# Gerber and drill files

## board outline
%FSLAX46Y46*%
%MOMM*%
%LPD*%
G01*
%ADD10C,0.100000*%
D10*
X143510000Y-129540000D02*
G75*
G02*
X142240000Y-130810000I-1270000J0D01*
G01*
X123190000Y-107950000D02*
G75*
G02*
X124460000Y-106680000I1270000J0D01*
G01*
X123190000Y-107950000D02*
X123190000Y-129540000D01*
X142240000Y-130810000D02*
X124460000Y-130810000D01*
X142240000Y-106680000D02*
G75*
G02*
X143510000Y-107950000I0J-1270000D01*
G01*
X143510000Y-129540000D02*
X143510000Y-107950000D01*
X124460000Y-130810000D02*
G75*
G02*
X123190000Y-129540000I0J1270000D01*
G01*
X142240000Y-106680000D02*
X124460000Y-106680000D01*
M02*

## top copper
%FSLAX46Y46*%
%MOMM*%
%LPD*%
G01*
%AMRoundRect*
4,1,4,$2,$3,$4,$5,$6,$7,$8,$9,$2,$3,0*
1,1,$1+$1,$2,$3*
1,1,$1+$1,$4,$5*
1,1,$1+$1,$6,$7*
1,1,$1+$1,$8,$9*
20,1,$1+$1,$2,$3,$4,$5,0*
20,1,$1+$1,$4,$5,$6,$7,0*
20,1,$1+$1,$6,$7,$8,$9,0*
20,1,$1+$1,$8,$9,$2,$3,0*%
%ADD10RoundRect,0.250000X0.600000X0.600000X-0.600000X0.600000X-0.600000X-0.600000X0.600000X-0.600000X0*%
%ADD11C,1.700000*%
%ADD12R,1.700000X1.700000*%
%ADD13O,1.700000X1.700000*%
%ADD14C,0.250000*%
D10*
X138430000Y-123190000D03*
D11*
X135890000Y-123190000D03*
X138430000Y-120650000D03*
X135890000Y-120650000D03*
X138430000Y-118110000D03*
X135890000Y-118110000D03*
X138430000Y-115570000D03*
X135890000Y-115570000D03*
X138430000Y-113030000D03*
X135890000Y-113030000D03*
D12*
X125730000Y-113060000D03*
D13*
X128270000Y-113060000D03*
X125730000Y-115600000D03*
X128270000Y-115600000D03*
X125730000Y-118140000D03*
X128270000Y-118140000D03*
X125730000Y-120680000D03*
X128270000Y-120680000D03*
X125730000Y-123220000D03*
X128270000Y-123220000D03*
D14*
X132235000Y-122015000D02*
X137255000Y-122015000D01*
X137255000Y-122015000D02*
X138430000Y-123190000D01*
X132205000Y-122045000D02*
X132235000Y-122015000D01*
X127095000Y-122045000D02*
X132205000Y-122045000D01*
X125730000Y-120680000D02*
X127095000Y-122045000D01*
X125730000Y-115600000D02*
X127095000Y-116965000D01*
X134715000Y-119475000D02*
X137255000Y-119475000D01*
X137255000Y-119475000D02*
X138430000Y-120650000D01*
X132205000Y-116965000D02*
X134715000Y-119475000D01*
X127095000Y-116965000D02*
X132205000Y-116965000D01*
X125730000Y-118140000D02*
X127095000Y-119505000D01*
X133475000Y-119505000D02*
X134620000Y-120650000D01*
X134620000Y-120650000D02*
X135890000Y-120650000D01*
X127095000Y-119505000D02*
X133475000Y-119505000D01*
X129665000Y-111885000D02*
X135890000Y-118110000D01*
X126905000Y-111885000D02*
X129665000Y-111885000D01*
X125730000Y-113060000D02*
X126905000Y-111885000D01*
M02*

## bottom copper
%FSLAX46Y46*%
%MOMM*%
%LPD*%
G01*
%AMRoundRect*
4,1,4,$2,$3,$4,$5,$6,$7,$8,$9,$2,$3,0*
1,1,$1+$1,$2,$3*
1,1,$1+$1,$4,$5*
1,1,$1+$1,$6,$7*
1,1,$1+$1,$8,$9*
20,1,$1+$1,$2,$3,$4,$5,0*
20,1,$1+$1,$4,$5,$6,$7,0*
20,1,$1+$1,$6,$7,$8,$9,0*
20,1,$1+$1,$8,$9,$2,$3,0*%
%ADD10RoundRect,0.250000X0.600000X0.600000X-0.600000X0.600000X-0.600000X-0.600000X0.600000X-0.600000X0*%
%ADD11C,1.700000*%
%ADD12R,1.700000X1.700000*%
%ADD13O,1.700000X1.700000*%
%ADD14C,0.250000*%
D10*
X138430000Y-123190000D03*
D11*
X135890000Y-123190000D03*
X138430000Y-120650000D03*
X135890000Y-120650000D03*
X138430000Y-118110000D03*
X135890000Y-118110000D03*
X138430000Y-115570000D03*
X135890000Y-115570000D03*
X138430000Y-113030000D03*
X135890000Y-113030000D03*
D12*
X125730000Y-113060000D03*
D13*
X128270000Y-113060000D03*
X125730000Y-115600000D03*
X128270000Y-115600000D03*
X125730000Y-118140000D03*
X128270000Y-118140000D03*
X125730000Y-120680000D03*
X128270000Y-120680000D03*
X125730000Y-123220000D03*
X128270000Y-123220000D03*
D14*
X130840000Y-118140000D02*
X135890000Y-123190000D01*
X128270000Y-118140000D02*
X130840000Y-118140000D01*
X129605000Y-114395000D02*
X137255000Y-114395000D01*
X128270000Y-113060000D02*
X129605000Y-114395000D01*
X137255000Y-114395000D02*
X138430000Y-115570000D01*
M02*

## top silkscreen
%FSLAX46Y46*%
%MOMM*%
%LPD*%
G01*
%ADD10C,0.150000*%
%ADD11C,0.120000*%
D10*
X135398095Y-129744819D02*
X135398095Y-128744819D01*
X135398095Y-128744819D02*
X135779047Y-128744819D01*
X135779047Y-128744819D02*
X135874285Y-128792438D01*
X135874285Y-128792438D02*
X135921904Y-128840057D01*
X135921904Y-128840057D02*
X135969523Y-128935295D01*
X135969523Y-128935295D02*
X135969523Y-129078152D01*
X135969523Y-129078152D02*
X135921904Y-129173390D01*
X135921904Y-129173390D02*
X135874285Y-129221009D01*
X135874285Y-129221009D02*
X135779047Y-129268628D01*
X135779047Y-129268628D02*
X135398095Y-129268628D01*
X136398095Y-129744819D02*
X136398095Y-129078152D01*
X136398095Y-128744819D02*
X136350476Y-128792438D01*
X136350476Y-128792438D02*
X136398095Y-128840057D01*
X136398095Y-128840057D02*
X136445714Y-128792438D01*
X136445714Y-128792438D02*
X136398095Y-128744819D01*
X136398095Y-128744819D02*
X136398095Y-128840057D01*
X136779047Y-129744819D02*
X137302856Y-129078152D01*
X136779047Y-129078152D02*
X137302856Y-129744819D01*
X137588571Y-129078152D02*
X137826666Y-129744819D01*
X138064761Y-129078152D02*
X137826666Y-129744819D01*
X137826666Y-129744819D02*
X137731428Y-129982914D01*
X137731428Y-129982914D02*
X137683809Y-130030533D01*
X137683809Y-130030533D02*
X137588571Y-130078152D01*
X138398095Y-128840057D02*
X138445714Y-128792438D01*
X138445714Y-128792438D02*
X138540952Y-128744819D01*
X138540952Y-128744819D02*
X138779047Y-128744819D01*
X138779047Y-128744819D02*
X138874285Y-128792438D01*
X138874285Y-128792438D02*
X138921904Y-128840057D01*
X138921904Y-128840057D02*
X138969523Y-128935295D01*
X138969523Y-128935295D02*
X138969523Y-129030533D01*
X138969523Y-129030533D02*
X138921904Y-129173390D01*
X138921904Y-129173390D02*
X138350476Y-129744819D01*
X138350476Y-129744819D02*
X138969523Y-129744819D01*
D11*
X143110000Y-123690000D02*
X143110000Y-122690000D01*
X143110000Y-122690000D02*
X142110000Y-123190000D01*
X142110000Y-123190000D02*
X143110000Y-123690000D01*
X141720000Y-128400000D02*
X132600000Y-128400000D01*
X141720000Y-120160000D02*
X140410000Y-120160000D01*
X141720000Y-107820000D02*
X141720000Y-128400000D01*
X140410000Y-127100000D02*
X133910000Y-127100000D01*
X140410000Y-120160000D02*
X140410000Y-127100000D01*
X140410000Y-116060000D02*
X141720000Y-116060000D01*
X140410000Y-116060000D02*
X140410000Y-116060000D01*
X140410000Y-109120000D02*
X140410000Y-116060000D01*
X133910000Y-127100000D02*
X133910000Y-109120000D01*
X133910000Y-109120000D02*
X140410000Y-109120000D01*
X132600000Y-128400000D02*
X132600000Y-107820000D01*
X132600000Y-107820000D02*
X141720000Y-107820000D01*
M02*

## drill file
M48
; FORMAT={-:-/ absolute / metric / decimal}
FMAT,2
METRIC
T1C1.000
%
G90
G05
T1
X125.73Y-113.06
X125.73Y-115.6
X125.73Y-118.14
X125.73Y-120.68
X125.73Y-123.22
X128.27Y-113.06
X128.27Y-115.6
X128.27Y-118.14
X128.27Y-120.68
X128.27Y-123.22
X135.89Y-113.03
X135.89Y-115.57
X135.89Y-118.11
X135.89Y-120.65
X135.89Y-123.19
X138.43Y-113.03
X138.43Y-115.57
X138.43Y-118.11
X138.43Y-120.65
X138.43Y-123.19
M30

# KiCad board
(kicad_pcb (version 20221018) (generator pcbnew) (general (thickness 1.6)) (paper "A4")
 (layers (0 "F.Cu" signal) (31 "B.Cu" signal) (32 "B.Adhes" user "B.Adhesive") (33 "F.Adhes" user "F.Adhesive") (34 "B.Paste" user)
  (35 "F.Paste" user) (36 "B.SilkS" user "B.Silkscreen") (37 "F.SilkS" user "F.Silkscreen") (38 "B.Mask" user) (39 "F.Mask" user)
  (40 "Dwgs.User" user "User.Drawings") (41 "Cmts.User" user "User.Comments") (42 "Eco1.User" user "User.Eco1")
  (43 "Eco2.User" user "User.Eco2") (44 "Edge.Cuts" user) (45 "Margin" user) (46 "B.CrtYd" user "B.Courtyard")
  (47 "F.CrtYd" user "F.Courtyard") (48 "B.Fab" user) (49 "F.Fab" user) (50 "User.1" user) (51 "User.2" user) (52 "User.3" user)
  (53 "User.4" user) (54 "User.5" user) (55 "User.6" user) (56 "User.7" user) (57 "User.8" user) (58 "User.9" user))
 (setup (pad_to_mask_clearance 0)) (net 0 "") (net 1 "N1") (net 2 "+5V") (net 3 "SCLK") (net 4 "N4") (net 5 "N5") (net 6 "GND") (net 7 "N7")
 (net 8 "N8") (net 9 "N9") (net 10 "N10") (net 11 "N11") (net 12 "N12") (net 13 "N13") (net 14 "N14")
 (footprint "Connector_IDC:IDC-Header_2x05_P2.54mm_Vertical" (layer "F.Cu") (at 138.43 123.19 180)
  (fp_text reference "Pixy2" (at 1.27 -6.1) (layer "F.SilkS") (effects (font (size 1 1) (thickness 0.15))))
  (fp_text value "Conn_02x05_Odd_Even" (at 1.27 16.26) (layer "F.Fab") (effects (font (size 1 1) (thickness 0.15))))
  (fp_line (start -4.68 -0.5) (end -4.68 0.5) (stroke (width 0.12) (type solid)) (layer "F.SilkS"))
  (fp_line (start -4.68 0.5) (end -3.68 0) (stroke (width 0.12) (type solid)) (layer "F.SilkS"))
  (fp_line (start -3.68 0) (end -4.68 -0.5) (stroke (width 0.12) (type solid)) (layer "F.SilkS"))
  (fp_line (start -3.29 -5.21) (end 5.83 -5.21) (stroke (width 0.12) (type solid)) (layer "F.SilkS"))
  (fp_line (start -3.29 3.03) (end -1.98 3.03) (stroke (width 0.12) (type solid)) (layer "F.SilkS"))
  (fp_line (start -3.29 15.37) (end -3.29 -5.21) (stroke (width 0.12) (type solid)) (layer "F.SilkS"))
  (fp_line (start -1.98 -3.91) (end 4.52 -3.91) (stroke (width 0.12) (type solid)) (layer "F.SilkS"))
  (fp_line (start -1.98 3.03) (end -1.98 -3.91) (stroke (width 0.12) (type solid)) (layer "F.SilkS"))
  (fp_line (start -1.98 7.13) (end -3.29 7.13) (stroke (width 0.12) (type solid)) (layer "F.SilkS"))
  (fp_line (start -1.98 7.13) (end -1.98 7.13) (stroke (width 0.12) (type solid)) (layer "F.SilkS"))
  (fp_line (start -1.98 14.07) (end -1.98 7.13) (stroke (width 0.12) (type solid)) (layer "F.SilkS"))
  (fp_line (start 4.52 -3.91) (end 4.52 14.07) (stroke (width 0.12) (type solid)) (layer "F.SilkS"))
  (fp_line (start 4.52 14.07) (end -1.98 14.07) (stroke (width 0.12) (type solid)) (layer "F.SilkS"))
  (fp_line (start 5.83 -5.21) (end 5.83 15.37) (stroke (width 0.12) (type solid)) (layer "F.SilkS"))
  (fp_line (start 5.83 15.37) (end -3.29 15.37) (stroke (width 0.12) (type solid)) (layer "F.SilkS"))
  (pad "1" thru_hole roundrect (at 0 0 180) (size 1.7 1.7) (drill 1) (layers "*.Cu" "*.Mask") (roundrect_rratio 0.147059) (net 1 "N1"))
  (pad "2" thru_hole circle (at 2.54 0 180) (size 1.7 1.7) (drill 1) (layers "*.Cu" "*.Mask") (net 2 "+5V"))
  (pad "3" thru_hole circle (at 0 2.54 180) (size 1.7 1.7) (drill 1) (layers "*.Cu" "*.Mask") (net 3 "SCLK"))
  (pad "4" thru_hole circle (at 2.54 2.54 180) (size 1.7 1.7) (drill 1) (layers "*.Cu" "*.Mask") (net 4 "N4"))
  (pad "5" thru_hole circle (at 0 5.08 180) (size 1.7 1.7) (drill 1) (layers "*.Cu" "*.Mask") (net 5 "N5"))
  (pad "6" thru_hole circle (at 2.54 5.08 180) (size 1.7 1.7) (drill 1) (layers "*.Cu" "*.Mask") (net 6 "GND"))
  (pad "7" thru_hole circle (at 0 7.62 180) (size 1.7 1.7) (drill 1) (layers "*.Cu" "*.Mask") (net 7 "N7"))
  (pad "8" thru_hole circle (at 2.54 7.62 180) (size 1.7 1.7) (drill 1) (layers "*.Cu" "*.Mask") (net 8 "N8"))
  (pad "9" thru_hole circle (at 0 10.16 180) (size 1.7 1.7) (drill 1) (layers "*.Cu" "*.Mask") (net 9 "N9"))
  (pad "10" thru_hole circle (at 2.54 10.16 180) (size 1.7 1.7) (drill 1) (layers "*.Cu" "*.Mask") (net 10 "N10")))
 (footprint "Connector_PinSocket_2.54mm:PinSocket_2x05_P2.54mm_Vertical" (layer "B.Cu") (at 125.73 113.06 180)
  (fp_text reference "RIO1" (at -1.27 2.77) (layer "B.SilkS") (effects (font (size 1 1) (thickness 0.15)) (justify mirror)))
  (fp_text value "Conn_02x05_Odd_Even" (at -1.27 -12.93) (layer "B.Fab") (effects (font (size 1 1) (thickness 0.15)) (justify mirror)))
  (pad "1" thru_hole rect (at 0 0 180) (size 1.7 1.7) (drill 1) (layers "*.Cu" "*.Mask") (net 6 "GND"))
  (pad "2" thru_hole oval (at -2.54 0 180) (size 1.7 1.7) (drill 1) (layers "*.Cu" "*.Mask") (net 7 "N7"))
  (pad "3" thru_hole oval (at 0 -2.54 180) (size 1.7 1.7) (drill 1) (layers "*.Cu" "*.Mask") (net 3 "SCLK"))
  (pad "4" thru_hole oval (at -2.54 -2.54 180) (size 1.7 1.7) (drill 1) (layers "*.Cu" "*.Mask") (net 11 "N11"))
  (pad "5" thru_hole oval (at 0 -5.08 180) (size 1.7 1.7) (drill 1) (layers "*.Cu" "*.Mask") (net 4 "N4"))
  (pad "6" thru_hole oval (at -2.54 -5.08 180) (size 1.7 1.7) (drill 1) (layers "*.Cu" "*.Mask") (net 2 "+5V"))
  (pad "7" thru_hole oval (at 0 -7.62 180) (size 1.7 1.7) (drill 1) (layers "*.Cu" "*.Mask") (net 1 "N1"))
  (pad "8" thru_hole oval (at -2.54 -7.62 180) (size 1.7 1.7) (drill 1) (layers "*.Cu" "*.Mask") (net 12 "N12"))
  (pad "9" thru_hole oval (at 0 -10.16 180) (size 1.7 1.7) (drill 1) (layers "*.Cu" "*.Mask") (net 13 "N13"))
  (pad "10" thru_hole oval (at -2.54 -10.16 180) (size 1.7 1.7) (drill 1) (layers "*.Cu" "*.Mask") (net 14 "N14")))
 (gr_arc (start 143.51 129.54) (mid 143.138026 130.438026) (end 142.24 130.81) (stroke (width 0.1) (type default)) (layer "Edge.Cuts"))
 (gr_arc (start 123.19 107.95) (mid 123.561974 107.051974) (end 124.46 106.68) (stroke (width 0.1) (type default)) (layer "Edge.Cuts"))
 (gr_line (start 123.19 107.95) (end 123.19 129.54) (stroke (width 0.1) (type default)) (layer "Edge.Cuts"))
 (gr_line (start 142.24 130.81) (end 124.46 130.81) (stroke (width 0.1) (type default)) (layer "Edge.Cuts"))
 (gr_arc (start 142.24 106.68) (mid 143.138026 107.051974) (end 143.51 107.95) (stroke (width 0.1) (type default)) (layer "Edge.Cuts"))
 (gr_line (start 143.51 129.54) (end 143.51 107.95) (stroke (width 0.1) (type default)) (layer "Edge.Cuts"))
 (gr_arc (start 124.46 130.81) (mid 123.561974 130.438026) (end 123.19 129.54) (stroke (width 0.1) (type default)) (layer "Edge.Cuts"))
 (gr_line (start 142.24 106.68) (end 124.46 106.68) (stroke (width 0.1) (type default)) (layer "Edge.Cuts"))
 (segment (start 132.235 122.015) (end 137.255 122.015) (width 0.25) (layer "F.Cu") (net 1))
 (segment (start 137.255 122.015) (end 138.43 123.19) (width 0.25) (layer "F.Cu") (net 1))
 (segment (start 132.205 122.045) (end 132.235 122.015) (width 0.25) (layer "F.Cu") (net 1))
 (segment (start 127.095 122.045) (end 132.205 122.045) (width 0.25) (layer "F.Cu") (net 1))
 (segment (start 125.73 120.68) (end 127.095 122.045) (width 0.25) (layer "F.Cu") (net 1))
 (segment (start 130.84 118.14) (end 135.89 123.19) (width 0.25) (layer "B.Cu") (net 2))
 (segment (start 128.27 118.14) (end 130.84 118.14) (width 0.25) (layer "B.Cu") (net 2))
 (segment (start 125.73 115.6) (end 127.095 116.965) (width 0.25) (layer "F.Cu") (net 3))
 (segment (start 134.715 119.475) (end 137.255 119.475) (width 0.25) (layer "F.Cu") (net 3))
 (segment (start 137.255 119.475) (end 138.43 120.65) (width 0.25) (layer "F.Cu") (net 3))
 (segment (start 132.205 116.965) (end 134.715 119.475) (width 0.25) (layer "F.Cu") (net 3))
 (segment (start 127.095 116.965) (end 132.205 116.965) (width 0.25) (layer "F.Cu") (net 3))
 (segment (start 125.73 118.14) (end 127.095 119.505) (width 0.25) (layer "F.Cu") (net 4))
 (segment (start 133.475 119.505) (end 134.62 120.65) (width 0.25) (layer "F.Cu") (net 4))
 (segment (start 134.62 120.65) (end 135.89 120.65) (width 0.25) (layer "F.Cu") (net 4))
 (segment (start 127.095 119.505) (end 133.475 119.505) (width 0.25) (layer "F.Cu") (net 4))
 (segment (start 129.665 111.885) (end 135.89 118.11) (width 0.25) (layer "F.Cu") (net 6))
 (segment (start 126.905 111.885) (end 129.665 111.885) (width 0.25) (layer "F.Cu") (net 6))
 (segment (start 125.73 113.06) (end 126.905 111.885) (width 0.25) (layer "F.Cu") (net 6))
 (segment (start 129.605 114.395) (end 137.255 114.395) (width 0.25) (layer "B.Cu") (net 7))
 (segment (start 128.27 113.06) (end 129.605 114.395) (width 0.25) (layer "B.Cu") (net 7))
 (segment (start 137.255 114.395) (end 138.43 115.57) (width 0.25) (layer "B.Cu") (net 7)))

